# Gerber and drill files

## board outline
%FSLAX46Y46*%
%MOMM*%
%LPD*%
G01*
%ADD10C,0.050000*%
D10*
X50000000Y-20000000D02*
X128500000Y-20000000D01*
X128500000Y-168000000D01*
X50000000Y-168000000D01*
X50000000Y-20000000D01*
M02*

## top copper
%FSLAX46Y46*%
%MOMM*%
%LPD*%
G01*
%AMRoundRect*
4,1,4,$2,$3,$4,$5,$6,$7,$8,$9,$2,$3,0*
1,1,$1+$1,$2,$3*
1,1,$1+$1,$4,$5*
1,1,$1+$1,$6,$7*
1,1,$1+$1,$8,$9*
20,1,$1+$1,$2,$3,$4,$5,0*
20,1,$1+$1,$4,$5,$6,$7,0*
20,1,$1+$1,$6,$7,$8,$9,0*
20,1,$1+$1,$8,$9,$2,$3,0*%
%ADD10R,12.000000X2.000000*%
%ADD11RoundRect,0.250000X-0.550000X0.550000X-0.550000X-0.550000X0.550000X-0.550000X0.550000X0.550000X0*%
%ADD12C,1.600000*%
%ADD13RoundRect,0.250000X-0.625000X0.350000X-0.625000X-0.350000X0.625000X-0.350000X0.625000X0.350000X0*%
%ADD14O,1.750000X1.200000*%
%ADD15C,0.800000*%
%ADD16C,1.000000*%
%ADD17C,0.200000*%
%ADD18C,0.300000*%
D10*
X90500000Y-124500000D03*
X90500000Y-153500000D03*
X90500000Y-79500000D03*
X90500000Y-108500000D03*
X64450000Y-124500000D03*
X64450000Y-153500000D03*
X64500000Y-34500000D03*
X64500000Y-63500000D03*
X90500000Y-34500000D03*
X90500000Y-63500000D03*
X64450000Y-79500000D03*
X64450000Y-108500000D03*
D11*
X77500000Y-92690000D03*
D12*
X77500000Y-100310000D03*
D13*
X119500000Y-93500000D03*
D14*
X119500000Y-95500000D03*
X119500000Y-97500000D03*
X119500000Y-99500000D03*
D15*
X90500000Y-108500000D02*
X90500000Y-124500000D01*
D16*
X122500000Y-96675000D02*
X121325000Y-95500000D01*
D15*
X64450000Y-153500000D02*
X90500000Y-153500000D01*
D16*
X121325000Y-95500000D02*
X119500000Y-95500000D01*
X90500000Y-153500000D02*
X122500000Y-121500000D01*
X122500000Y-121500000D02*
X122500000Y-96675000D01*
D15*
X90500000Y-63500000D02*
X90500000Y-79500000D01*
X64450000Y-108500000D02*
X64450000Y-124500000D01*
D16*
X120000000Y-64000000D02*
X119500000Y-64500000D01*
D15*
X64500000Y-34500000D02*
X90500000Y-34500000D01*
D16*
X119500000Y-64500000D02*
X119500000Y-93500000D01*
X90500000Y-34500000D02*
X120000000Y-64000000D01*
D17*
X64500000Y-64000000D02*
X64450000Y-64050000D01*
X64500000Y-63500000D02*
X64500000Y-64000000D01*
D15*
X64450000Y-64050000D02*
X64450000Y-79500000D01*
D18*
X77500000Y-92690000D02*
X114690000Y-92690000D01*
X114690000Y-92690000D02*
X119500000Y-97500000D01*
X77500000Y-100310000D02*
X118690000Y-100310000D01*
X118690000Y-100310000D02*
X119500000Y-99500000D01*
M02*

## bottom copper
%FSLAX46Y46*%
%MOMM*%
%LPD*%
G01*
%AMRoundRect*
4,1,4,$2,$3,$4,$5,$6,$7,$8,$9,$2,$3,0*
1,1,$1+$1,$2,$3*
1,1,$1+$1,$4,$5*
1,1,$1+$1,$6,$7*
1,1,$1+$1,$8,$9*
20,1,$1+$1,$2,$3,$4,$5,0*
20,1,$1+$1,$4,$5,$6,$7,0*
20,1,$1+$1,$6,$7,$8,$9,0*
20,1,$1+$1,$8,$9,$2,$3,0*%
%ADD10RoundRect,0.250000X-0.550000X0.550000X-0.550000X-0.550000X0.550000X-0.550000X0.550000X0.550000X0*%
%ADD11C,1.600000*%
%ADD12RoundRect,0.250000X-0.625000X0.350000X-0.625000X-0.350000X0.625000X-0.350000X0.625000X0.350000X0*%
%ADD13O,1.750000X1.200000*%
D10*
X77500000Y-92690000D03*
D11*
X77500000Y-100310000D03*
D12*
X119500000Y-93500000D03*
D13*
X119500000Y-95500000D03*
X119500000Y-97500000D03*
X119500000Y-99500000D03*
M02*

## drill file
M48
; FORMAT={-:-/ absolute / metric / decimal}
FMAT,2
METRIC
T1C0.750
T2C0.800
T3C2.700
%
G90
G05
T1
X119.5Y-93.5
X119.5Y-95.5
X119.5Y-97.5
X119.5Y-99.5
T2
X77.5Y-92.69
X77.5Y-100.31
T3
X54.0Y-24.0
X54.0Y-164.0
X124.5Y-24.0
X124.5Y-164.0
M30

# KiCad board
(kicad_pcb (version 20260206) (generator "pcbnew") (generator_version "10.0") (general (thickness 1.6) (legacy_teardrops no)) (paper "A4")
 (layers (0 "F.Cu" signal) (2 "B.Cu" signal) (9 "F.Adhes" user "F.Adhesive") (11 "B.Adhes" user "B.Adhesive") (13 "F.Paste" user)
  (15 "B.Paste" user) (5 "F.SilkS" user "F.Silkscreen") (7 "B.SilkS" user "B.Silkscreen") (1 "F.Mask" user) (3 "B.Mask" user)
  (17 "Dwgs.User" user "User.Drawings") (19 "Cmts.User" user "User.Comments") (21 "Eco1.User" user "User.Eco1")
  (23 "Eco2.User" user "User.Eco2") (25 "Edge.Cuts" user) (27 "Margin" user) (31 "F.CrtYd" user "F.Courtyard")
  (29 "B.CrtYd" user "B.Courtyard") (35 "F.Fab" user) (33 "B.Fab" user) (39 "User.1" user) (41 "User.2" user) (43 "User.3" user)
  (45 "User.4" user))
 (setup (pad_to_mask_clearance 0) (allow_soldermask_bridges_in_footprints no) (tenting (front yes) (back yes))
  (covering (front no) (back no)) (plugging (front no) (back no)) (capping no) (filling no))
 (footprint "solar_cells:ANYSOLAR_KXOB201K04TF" (layer "F.Cu") (at 90.5 139 180)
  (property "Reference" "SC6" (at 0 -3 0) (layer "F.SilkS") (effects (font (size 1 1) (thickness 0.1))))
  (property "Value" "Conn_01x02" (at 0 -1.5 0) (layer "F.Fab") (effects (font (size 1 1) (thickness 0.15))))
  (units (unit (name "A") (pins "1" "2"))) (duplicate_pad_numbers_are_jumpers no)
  (pad "1" smd rect (at 0 14.5 180) (size 12 2) (layers "F.Cu" "F.Mask" "F.Paste") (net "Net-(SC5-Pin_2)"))
  (pad "2" smd rect (at 0 -14.5 180) (size 12 2) (layers "F.Cu" "F.Mask" "F.Paste") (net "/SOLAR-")))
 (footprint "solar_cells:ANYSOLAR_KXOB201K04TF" (layer "F.Cu") (at 90.5 94 180)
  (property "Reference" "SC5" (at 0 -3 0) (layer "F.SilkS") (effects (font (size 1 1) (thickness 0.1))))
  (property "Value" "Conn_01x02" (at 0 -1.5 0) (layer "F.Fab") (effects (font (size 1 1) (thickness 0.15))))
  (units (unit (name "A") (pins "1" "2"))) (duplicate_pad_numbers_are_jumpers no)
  (pad "1" smd rect (at 0 14.5 180) (size 12 2) (layers "F.Cu" "F.Mask" "F.Paste") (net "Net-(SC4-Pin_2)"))
  (pad "2" smd rect (at 0 -14.5 180) (size 12 2) (layers "F.Cu" "F.Mask" "F.Paste") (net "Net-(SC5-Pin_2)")))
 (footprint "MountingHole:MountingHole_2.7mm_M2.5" (layer "F.Cu") (at 54 164)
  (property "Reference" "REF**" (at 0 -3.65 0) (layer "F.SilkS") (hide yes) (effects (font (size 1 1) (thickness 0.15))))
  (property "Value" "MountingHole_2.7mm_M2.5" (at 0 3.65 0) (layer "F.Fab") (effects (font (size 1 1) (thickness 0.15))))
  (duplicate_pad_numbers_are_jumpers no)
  (pad "" np_thru_hole circle (at 0 0) (size 2.7 2.7) (drill 2.7) (layers "*.Cu" "*.Mask")))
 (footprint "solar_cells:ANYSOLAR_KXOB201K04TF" (layer "F.Cu") (at 64.45 139 180)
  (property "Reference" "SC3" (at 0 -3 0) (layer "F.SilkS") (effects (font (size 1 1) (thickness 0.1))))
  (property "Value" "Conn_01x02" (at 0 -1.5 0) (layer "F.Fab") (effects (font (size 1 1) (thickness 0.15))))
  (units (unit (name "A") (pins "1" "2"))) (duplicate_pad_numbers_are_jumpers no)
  (pad "1" smd rect (at 0 14.5 180) (size 12 2) (layers "F.Cu" "F.Mask" "F.Paste") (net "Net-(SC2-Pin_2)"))
  (pad "2" smd rect (at 0 -14.5 180) (size 12 2) (layers "F.Cu" "F.Mask" "F.Paste") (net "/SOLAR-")))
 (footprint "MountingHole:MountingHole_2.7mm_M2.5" (layer "F.Cu") (at 124.5 164)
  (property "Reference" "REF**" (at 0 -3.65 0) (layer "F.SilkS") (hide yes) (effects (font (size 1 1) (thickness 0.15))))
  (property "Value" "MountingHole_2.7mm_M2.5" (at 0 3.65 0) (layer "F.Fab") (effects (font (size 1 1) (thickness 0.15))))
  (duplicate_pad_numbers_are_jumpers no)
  (pad "" np_thru_hole circle (at 0 0) (size 2.7 2.7) (drill 2.7) (layers "*.Cu" "*.Mask")))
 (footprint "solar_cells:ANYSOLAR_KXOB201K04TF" (layer "F.Cu") (at 64.5 49 180)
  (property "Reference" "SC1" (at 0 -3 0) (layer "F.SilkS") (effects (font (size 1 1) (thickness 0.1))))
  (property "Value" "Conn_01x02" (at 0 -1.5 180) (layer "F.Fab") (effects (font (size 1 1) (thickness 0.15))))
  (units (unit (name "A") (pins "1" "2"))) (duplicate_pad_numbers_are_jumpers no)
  (pad "1" smd rect (at 0 14.5 180) (size 12 2) (layers "F.Cu" "F.Mask" "F.Paste") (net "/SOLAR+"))
  (pad "2" smd rect (at 0 -14.5 180) (size 12 2) (layers "F.Cu" "F.Mask" "F.Paste") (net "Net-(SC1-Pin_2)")))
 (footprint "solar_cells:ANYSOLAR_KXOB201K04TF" (layer "F.Cu") (at 90.5 49 180)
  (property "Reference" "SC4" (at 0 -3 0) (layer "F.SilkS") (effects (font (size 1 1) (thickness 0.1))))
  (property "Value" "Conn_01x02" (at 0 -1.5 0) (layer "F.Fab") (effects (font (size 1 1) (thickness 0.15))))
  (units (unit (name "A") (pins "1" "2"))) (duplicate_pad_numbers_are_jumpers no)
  (pad "1" smd rect (at 0 14.5 180) (size 12 2) (layers "F.Cu" "F.Mask" "F.Paste") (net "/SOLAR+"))
  (pad "2" smd rect (at 0 -14.5 180) (size 12 2) (layers "F.Cu" "F.Mask" "F.Paste") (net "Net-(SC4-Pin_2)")))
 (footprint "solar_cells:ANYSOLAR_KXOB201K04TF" (layer "F.Cu") (at 64.45 94 180)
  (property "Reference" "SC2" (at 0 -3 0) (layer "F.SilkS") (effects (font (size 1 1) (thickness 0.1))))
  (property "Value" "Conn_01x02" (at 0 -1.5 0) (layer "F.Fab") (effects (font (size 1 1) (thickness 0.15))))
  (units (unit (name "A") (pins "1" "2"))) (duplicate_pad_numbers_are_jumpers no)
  (pad "1" smd rect (at 0 14.5 180) (size 12 2) (layers "F.Cu" "F.Mask" "F.Paste") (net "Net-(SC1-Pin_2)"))
  (pad "2" smd rect (at 0 -14.5 180) (size 12 2) (layers "F.Cu" "F.Mask" "F.Paste") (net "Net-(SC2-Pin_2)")))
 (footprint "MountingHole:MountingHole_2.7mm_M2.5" (layer "F.Cu") (at 124.5 24)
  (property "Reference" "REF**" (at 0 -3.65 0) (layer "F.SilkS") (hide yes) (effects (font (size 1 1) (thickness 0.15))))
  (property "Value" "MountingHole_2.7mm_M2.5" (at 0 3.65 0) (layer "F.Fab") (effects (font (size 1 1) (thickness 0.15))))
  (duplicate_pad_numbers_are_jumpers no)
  (pad "" np_thru_hole circle (at 0 0) (size 2.7 2.7) (drill 2.7) (layers "*.Cu" "*.Mask")))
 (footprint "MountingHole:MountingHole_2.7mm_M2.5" (layer "F.Cu") (at 54 24)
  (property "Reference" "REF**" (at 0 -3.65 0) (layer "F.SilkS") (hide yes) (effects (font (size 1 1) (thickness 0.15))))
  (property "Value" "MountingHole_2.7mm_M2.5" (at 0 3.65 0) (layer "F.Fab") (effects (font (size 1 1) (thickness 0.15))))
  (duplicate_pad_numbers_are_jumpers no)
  (pad "" np_thru_hole circle (at 0 0) (size 2.7 2.7) (drill 2.7) (layers "*.Cu" "*.Mask")))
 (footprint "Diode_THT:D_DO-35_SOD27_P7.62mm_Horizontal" (layer "B.Cu") (at 77.5 92.69 -90)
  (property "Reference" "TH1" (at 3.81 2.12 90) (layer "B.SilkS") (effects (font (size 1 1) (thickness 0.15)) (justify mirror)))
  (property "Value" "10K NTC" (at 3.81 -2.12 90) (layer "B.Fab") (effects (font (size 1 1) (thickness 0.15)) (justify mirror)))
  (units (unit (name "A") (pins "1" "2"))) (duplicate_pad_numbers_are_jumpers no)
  (pad "1" thru_hole roundrect (at 0 0 270) (size 1.6 1.6) (drill 0.8) (layers "*.Cu" "*.Mask") (remove_unused_layers no)
   (roundrect_rratio 0.15625) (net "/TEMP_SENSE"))
  (pad "2" thru_hole circle (at 7.62 0 270) (size 1.6 1.6) (drill 0.8) (layers "*.Cu" "*.Mask") (remove_unused_layers no)
   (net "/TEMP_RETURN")))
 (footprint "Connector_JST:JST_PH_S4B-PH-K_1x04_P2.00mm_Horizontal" (layer "B.Cu") (at 119.5 93.5 -90)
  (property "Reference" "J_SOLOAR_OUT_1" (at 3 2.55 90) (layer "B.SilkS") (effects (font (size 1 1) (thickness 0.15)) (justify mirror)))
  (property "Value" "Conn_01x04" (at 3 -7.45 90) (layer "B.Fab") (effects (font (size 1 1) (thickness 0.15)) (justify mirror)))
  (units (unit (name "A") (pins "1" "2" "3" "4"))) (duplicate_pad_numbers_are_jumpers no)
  (pad "1" thru_hole roundrect (at 0 0 270) (size 1.2 1.75) (drill 0.75) (layers "*.Cu" "*.Mask") (remove_unused_layers no)
   (roundrect_rratio 0.208333) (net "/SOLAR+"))
  (pad "2" thru_hole oval (at 2 0 270) (size 1.2 1.75) (drill 0.75) (layers "*.Cu" "*.Mask") (remove_unused_layers no) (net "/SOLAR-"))
  (pad "3" thru_hole oval (at 4 0 270) (size 1.2 1.75) (drill 0.75) (layers "*.Cu" "*.Mask") (remove_unused_layers no) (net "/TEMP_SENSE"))
  (pad "4" thru_hole oval (at 6 0 270) (size 1.2 1.75) (drill 0.75) (layers "*.Cu" "*.Mask") (remove_unused_layers no) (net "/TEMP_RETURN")))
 (gr_rect (start 50 20) (end 128.5 168) (stroke (width 0.05) (type default)) (fill no) (layer "Edge.Cuts"))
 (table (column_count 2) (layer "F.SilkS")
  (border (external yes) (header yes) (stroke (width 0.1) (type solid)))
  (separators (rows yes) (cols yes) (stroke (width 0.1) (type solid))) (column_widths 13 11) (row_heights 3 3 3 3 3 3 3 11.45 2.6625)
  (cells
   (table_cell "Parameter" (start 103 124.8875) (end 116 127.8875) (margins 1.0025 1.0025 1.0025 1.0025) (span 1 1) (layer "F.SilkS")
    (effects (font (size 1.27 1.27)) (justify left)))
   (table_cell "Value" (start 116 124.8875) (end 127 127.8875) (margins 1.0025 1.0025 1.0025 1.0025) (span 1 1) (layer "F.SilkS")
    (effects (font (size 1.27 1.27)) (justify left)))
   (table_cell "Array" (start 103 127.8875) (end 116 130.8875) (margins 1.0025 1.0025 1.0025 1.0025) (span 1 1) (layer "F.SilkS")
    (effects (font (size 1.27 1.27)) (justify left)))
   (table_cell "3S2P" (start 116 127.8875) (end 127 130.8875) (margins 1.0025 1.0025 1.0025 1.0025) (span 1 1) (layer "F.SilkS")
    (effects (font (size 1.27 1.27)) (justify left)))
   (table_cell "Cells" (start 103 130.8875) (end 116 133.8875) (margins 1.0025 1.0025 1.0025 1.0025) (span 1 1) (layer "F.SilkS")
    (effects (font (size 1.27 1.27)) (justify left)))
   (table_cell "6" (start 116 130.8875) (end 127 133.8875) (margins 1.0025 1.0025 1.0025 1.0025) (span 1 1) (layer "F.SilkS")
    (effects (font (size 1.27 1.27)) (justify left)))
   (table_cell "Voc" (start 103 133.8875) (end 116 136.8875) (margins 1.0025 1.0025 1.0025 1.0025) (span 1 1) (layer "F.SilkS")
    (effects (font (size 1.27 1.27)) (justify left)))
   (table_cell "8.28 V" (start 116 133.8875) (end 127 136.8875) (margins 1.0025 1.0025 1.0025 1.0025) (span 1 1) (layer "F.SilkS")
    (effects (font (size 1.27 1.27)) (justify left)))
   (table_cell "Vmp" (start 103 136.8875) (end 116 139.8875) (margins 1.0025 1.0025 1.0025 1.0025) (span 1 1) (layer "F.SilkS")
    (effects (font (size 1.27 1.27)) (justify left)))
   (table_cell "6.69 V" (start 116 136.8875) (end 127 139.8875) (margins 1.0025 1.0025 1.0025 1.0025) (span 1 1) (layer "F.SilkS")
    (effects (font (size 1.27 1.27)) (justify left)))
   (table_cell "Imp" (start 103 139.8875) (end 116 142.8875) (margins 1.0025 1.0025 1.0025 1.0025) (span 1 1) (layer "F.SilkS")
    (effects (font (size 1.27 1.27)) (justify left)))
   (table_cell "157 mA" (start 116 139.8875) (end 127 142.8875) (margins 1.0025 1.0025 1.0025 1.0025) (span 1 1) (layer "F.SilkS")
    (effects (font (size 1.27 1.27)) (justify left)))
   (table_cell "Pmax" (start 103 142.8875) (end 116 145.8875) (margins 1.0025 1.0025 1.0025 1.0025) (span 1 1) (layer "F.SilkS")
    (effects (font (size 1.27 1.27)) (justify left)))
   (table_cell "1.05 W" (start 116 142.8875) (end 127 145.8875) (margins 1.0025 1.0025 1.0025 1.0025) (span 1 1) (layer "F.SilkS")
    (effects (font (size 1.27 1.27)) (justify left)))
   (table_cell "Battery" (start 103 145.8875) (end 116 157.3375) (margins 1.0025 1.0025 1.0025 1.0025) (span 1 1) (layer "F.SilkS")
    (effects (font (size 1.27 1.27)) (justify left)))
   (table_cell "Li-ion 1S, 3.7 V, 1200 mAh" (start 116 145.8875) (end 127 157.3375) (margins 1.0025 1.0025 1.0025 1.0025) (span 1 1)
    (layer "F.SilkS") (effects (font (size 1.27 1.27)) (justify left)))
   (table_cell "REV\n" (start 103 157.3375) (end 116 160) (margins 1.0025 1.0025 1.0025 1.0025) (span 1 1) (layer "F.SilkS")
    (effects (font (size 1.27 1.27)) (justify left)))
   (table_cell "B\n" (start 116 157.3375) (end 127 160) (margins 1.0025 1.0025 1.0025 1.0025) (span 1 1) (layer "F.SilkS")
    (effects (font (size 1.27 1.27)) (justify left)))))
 (segment (start 90.5 108.5) (end 90.5 124.5) (width 0.8) (layer "F.Cu") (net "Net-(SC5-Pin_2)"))
 (segment (start 122.5 96.675) (end 121.325 95.5) (width 1) (layer "F.Cu") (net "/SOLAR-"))
 (segment (start 64.45 153.5) (end 90.5 153.5) (width 0.8) (layer "F.Cu") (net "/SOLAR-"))
 (segment (start 121.325 95.5) (end 119.5 95.5) (width 1) (layer "F.Cu") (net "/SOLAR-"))
 (segment (start 90.5 153.5) (end 122.5 121.5) (width 1) (layer "F.Cu") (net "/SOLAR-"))
 (segment (start 122.5 121.5) (end 122.5 96.675) (width 1) (layer "F.Cu") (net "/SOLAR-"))
 (segment (start 90.5 63.5) (end 90.5 79.5) (width 0.8) (layer "F.Cu") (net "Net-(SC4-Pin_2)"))
 (segment (start 64.45 108.5) (end 64.45 124.5) (width 0.8) (layer "F.Cu") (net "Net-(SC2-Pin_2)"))
 (segment (start 120 64) (end 119.5 64.5) (width 1) (layer "F.Cu") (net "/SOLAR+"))
 (segment (start 64.5 34.5) (end 90.5 34.5) (width 0.8) (layer "F.Cu") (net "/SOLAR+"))
 (segment (start 119.5 64.5) (end 119.5 93.5) (width 1) (layer "F.Cu") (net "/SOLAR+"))
 (segment (start 90.5 34.5) (end 120 64) (width 1) (layer "F.Cu") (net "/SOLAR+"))
 (segment (start 64.5 64) (end 64.45 64.05) (width 0.2) (layer "F.Cu") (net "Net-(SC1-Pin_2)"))
 (segment (start 64.5 63.5) (end 64.5 64) (width 0.2) (layer "F.Cu") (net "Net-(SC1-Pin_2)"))
 (segment (start 64.45 64.05) (end 64.45 79.5) (width 0.8) (layer "F.Cu") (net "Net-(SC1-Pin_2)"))
 (segment (start 77.5 92.69) (end 114.69 92.69) (width 0.3) (layer "F.Cu") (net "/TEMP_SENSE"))
 (segment (start 114.69 92.69) (end 119.5 97.5) (width 0.3) (layer "F.Cu") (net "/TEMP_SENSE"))
 (segment (start 77.5 100.31) (end 118.69 100.31) (width 0.3) (layer "F.Cu") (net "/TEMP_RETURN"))
 (segment (start 118.69 100.31) (end 119.5 99.5) (width 0.3) (layer "F.Cu") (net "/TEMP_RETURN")))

